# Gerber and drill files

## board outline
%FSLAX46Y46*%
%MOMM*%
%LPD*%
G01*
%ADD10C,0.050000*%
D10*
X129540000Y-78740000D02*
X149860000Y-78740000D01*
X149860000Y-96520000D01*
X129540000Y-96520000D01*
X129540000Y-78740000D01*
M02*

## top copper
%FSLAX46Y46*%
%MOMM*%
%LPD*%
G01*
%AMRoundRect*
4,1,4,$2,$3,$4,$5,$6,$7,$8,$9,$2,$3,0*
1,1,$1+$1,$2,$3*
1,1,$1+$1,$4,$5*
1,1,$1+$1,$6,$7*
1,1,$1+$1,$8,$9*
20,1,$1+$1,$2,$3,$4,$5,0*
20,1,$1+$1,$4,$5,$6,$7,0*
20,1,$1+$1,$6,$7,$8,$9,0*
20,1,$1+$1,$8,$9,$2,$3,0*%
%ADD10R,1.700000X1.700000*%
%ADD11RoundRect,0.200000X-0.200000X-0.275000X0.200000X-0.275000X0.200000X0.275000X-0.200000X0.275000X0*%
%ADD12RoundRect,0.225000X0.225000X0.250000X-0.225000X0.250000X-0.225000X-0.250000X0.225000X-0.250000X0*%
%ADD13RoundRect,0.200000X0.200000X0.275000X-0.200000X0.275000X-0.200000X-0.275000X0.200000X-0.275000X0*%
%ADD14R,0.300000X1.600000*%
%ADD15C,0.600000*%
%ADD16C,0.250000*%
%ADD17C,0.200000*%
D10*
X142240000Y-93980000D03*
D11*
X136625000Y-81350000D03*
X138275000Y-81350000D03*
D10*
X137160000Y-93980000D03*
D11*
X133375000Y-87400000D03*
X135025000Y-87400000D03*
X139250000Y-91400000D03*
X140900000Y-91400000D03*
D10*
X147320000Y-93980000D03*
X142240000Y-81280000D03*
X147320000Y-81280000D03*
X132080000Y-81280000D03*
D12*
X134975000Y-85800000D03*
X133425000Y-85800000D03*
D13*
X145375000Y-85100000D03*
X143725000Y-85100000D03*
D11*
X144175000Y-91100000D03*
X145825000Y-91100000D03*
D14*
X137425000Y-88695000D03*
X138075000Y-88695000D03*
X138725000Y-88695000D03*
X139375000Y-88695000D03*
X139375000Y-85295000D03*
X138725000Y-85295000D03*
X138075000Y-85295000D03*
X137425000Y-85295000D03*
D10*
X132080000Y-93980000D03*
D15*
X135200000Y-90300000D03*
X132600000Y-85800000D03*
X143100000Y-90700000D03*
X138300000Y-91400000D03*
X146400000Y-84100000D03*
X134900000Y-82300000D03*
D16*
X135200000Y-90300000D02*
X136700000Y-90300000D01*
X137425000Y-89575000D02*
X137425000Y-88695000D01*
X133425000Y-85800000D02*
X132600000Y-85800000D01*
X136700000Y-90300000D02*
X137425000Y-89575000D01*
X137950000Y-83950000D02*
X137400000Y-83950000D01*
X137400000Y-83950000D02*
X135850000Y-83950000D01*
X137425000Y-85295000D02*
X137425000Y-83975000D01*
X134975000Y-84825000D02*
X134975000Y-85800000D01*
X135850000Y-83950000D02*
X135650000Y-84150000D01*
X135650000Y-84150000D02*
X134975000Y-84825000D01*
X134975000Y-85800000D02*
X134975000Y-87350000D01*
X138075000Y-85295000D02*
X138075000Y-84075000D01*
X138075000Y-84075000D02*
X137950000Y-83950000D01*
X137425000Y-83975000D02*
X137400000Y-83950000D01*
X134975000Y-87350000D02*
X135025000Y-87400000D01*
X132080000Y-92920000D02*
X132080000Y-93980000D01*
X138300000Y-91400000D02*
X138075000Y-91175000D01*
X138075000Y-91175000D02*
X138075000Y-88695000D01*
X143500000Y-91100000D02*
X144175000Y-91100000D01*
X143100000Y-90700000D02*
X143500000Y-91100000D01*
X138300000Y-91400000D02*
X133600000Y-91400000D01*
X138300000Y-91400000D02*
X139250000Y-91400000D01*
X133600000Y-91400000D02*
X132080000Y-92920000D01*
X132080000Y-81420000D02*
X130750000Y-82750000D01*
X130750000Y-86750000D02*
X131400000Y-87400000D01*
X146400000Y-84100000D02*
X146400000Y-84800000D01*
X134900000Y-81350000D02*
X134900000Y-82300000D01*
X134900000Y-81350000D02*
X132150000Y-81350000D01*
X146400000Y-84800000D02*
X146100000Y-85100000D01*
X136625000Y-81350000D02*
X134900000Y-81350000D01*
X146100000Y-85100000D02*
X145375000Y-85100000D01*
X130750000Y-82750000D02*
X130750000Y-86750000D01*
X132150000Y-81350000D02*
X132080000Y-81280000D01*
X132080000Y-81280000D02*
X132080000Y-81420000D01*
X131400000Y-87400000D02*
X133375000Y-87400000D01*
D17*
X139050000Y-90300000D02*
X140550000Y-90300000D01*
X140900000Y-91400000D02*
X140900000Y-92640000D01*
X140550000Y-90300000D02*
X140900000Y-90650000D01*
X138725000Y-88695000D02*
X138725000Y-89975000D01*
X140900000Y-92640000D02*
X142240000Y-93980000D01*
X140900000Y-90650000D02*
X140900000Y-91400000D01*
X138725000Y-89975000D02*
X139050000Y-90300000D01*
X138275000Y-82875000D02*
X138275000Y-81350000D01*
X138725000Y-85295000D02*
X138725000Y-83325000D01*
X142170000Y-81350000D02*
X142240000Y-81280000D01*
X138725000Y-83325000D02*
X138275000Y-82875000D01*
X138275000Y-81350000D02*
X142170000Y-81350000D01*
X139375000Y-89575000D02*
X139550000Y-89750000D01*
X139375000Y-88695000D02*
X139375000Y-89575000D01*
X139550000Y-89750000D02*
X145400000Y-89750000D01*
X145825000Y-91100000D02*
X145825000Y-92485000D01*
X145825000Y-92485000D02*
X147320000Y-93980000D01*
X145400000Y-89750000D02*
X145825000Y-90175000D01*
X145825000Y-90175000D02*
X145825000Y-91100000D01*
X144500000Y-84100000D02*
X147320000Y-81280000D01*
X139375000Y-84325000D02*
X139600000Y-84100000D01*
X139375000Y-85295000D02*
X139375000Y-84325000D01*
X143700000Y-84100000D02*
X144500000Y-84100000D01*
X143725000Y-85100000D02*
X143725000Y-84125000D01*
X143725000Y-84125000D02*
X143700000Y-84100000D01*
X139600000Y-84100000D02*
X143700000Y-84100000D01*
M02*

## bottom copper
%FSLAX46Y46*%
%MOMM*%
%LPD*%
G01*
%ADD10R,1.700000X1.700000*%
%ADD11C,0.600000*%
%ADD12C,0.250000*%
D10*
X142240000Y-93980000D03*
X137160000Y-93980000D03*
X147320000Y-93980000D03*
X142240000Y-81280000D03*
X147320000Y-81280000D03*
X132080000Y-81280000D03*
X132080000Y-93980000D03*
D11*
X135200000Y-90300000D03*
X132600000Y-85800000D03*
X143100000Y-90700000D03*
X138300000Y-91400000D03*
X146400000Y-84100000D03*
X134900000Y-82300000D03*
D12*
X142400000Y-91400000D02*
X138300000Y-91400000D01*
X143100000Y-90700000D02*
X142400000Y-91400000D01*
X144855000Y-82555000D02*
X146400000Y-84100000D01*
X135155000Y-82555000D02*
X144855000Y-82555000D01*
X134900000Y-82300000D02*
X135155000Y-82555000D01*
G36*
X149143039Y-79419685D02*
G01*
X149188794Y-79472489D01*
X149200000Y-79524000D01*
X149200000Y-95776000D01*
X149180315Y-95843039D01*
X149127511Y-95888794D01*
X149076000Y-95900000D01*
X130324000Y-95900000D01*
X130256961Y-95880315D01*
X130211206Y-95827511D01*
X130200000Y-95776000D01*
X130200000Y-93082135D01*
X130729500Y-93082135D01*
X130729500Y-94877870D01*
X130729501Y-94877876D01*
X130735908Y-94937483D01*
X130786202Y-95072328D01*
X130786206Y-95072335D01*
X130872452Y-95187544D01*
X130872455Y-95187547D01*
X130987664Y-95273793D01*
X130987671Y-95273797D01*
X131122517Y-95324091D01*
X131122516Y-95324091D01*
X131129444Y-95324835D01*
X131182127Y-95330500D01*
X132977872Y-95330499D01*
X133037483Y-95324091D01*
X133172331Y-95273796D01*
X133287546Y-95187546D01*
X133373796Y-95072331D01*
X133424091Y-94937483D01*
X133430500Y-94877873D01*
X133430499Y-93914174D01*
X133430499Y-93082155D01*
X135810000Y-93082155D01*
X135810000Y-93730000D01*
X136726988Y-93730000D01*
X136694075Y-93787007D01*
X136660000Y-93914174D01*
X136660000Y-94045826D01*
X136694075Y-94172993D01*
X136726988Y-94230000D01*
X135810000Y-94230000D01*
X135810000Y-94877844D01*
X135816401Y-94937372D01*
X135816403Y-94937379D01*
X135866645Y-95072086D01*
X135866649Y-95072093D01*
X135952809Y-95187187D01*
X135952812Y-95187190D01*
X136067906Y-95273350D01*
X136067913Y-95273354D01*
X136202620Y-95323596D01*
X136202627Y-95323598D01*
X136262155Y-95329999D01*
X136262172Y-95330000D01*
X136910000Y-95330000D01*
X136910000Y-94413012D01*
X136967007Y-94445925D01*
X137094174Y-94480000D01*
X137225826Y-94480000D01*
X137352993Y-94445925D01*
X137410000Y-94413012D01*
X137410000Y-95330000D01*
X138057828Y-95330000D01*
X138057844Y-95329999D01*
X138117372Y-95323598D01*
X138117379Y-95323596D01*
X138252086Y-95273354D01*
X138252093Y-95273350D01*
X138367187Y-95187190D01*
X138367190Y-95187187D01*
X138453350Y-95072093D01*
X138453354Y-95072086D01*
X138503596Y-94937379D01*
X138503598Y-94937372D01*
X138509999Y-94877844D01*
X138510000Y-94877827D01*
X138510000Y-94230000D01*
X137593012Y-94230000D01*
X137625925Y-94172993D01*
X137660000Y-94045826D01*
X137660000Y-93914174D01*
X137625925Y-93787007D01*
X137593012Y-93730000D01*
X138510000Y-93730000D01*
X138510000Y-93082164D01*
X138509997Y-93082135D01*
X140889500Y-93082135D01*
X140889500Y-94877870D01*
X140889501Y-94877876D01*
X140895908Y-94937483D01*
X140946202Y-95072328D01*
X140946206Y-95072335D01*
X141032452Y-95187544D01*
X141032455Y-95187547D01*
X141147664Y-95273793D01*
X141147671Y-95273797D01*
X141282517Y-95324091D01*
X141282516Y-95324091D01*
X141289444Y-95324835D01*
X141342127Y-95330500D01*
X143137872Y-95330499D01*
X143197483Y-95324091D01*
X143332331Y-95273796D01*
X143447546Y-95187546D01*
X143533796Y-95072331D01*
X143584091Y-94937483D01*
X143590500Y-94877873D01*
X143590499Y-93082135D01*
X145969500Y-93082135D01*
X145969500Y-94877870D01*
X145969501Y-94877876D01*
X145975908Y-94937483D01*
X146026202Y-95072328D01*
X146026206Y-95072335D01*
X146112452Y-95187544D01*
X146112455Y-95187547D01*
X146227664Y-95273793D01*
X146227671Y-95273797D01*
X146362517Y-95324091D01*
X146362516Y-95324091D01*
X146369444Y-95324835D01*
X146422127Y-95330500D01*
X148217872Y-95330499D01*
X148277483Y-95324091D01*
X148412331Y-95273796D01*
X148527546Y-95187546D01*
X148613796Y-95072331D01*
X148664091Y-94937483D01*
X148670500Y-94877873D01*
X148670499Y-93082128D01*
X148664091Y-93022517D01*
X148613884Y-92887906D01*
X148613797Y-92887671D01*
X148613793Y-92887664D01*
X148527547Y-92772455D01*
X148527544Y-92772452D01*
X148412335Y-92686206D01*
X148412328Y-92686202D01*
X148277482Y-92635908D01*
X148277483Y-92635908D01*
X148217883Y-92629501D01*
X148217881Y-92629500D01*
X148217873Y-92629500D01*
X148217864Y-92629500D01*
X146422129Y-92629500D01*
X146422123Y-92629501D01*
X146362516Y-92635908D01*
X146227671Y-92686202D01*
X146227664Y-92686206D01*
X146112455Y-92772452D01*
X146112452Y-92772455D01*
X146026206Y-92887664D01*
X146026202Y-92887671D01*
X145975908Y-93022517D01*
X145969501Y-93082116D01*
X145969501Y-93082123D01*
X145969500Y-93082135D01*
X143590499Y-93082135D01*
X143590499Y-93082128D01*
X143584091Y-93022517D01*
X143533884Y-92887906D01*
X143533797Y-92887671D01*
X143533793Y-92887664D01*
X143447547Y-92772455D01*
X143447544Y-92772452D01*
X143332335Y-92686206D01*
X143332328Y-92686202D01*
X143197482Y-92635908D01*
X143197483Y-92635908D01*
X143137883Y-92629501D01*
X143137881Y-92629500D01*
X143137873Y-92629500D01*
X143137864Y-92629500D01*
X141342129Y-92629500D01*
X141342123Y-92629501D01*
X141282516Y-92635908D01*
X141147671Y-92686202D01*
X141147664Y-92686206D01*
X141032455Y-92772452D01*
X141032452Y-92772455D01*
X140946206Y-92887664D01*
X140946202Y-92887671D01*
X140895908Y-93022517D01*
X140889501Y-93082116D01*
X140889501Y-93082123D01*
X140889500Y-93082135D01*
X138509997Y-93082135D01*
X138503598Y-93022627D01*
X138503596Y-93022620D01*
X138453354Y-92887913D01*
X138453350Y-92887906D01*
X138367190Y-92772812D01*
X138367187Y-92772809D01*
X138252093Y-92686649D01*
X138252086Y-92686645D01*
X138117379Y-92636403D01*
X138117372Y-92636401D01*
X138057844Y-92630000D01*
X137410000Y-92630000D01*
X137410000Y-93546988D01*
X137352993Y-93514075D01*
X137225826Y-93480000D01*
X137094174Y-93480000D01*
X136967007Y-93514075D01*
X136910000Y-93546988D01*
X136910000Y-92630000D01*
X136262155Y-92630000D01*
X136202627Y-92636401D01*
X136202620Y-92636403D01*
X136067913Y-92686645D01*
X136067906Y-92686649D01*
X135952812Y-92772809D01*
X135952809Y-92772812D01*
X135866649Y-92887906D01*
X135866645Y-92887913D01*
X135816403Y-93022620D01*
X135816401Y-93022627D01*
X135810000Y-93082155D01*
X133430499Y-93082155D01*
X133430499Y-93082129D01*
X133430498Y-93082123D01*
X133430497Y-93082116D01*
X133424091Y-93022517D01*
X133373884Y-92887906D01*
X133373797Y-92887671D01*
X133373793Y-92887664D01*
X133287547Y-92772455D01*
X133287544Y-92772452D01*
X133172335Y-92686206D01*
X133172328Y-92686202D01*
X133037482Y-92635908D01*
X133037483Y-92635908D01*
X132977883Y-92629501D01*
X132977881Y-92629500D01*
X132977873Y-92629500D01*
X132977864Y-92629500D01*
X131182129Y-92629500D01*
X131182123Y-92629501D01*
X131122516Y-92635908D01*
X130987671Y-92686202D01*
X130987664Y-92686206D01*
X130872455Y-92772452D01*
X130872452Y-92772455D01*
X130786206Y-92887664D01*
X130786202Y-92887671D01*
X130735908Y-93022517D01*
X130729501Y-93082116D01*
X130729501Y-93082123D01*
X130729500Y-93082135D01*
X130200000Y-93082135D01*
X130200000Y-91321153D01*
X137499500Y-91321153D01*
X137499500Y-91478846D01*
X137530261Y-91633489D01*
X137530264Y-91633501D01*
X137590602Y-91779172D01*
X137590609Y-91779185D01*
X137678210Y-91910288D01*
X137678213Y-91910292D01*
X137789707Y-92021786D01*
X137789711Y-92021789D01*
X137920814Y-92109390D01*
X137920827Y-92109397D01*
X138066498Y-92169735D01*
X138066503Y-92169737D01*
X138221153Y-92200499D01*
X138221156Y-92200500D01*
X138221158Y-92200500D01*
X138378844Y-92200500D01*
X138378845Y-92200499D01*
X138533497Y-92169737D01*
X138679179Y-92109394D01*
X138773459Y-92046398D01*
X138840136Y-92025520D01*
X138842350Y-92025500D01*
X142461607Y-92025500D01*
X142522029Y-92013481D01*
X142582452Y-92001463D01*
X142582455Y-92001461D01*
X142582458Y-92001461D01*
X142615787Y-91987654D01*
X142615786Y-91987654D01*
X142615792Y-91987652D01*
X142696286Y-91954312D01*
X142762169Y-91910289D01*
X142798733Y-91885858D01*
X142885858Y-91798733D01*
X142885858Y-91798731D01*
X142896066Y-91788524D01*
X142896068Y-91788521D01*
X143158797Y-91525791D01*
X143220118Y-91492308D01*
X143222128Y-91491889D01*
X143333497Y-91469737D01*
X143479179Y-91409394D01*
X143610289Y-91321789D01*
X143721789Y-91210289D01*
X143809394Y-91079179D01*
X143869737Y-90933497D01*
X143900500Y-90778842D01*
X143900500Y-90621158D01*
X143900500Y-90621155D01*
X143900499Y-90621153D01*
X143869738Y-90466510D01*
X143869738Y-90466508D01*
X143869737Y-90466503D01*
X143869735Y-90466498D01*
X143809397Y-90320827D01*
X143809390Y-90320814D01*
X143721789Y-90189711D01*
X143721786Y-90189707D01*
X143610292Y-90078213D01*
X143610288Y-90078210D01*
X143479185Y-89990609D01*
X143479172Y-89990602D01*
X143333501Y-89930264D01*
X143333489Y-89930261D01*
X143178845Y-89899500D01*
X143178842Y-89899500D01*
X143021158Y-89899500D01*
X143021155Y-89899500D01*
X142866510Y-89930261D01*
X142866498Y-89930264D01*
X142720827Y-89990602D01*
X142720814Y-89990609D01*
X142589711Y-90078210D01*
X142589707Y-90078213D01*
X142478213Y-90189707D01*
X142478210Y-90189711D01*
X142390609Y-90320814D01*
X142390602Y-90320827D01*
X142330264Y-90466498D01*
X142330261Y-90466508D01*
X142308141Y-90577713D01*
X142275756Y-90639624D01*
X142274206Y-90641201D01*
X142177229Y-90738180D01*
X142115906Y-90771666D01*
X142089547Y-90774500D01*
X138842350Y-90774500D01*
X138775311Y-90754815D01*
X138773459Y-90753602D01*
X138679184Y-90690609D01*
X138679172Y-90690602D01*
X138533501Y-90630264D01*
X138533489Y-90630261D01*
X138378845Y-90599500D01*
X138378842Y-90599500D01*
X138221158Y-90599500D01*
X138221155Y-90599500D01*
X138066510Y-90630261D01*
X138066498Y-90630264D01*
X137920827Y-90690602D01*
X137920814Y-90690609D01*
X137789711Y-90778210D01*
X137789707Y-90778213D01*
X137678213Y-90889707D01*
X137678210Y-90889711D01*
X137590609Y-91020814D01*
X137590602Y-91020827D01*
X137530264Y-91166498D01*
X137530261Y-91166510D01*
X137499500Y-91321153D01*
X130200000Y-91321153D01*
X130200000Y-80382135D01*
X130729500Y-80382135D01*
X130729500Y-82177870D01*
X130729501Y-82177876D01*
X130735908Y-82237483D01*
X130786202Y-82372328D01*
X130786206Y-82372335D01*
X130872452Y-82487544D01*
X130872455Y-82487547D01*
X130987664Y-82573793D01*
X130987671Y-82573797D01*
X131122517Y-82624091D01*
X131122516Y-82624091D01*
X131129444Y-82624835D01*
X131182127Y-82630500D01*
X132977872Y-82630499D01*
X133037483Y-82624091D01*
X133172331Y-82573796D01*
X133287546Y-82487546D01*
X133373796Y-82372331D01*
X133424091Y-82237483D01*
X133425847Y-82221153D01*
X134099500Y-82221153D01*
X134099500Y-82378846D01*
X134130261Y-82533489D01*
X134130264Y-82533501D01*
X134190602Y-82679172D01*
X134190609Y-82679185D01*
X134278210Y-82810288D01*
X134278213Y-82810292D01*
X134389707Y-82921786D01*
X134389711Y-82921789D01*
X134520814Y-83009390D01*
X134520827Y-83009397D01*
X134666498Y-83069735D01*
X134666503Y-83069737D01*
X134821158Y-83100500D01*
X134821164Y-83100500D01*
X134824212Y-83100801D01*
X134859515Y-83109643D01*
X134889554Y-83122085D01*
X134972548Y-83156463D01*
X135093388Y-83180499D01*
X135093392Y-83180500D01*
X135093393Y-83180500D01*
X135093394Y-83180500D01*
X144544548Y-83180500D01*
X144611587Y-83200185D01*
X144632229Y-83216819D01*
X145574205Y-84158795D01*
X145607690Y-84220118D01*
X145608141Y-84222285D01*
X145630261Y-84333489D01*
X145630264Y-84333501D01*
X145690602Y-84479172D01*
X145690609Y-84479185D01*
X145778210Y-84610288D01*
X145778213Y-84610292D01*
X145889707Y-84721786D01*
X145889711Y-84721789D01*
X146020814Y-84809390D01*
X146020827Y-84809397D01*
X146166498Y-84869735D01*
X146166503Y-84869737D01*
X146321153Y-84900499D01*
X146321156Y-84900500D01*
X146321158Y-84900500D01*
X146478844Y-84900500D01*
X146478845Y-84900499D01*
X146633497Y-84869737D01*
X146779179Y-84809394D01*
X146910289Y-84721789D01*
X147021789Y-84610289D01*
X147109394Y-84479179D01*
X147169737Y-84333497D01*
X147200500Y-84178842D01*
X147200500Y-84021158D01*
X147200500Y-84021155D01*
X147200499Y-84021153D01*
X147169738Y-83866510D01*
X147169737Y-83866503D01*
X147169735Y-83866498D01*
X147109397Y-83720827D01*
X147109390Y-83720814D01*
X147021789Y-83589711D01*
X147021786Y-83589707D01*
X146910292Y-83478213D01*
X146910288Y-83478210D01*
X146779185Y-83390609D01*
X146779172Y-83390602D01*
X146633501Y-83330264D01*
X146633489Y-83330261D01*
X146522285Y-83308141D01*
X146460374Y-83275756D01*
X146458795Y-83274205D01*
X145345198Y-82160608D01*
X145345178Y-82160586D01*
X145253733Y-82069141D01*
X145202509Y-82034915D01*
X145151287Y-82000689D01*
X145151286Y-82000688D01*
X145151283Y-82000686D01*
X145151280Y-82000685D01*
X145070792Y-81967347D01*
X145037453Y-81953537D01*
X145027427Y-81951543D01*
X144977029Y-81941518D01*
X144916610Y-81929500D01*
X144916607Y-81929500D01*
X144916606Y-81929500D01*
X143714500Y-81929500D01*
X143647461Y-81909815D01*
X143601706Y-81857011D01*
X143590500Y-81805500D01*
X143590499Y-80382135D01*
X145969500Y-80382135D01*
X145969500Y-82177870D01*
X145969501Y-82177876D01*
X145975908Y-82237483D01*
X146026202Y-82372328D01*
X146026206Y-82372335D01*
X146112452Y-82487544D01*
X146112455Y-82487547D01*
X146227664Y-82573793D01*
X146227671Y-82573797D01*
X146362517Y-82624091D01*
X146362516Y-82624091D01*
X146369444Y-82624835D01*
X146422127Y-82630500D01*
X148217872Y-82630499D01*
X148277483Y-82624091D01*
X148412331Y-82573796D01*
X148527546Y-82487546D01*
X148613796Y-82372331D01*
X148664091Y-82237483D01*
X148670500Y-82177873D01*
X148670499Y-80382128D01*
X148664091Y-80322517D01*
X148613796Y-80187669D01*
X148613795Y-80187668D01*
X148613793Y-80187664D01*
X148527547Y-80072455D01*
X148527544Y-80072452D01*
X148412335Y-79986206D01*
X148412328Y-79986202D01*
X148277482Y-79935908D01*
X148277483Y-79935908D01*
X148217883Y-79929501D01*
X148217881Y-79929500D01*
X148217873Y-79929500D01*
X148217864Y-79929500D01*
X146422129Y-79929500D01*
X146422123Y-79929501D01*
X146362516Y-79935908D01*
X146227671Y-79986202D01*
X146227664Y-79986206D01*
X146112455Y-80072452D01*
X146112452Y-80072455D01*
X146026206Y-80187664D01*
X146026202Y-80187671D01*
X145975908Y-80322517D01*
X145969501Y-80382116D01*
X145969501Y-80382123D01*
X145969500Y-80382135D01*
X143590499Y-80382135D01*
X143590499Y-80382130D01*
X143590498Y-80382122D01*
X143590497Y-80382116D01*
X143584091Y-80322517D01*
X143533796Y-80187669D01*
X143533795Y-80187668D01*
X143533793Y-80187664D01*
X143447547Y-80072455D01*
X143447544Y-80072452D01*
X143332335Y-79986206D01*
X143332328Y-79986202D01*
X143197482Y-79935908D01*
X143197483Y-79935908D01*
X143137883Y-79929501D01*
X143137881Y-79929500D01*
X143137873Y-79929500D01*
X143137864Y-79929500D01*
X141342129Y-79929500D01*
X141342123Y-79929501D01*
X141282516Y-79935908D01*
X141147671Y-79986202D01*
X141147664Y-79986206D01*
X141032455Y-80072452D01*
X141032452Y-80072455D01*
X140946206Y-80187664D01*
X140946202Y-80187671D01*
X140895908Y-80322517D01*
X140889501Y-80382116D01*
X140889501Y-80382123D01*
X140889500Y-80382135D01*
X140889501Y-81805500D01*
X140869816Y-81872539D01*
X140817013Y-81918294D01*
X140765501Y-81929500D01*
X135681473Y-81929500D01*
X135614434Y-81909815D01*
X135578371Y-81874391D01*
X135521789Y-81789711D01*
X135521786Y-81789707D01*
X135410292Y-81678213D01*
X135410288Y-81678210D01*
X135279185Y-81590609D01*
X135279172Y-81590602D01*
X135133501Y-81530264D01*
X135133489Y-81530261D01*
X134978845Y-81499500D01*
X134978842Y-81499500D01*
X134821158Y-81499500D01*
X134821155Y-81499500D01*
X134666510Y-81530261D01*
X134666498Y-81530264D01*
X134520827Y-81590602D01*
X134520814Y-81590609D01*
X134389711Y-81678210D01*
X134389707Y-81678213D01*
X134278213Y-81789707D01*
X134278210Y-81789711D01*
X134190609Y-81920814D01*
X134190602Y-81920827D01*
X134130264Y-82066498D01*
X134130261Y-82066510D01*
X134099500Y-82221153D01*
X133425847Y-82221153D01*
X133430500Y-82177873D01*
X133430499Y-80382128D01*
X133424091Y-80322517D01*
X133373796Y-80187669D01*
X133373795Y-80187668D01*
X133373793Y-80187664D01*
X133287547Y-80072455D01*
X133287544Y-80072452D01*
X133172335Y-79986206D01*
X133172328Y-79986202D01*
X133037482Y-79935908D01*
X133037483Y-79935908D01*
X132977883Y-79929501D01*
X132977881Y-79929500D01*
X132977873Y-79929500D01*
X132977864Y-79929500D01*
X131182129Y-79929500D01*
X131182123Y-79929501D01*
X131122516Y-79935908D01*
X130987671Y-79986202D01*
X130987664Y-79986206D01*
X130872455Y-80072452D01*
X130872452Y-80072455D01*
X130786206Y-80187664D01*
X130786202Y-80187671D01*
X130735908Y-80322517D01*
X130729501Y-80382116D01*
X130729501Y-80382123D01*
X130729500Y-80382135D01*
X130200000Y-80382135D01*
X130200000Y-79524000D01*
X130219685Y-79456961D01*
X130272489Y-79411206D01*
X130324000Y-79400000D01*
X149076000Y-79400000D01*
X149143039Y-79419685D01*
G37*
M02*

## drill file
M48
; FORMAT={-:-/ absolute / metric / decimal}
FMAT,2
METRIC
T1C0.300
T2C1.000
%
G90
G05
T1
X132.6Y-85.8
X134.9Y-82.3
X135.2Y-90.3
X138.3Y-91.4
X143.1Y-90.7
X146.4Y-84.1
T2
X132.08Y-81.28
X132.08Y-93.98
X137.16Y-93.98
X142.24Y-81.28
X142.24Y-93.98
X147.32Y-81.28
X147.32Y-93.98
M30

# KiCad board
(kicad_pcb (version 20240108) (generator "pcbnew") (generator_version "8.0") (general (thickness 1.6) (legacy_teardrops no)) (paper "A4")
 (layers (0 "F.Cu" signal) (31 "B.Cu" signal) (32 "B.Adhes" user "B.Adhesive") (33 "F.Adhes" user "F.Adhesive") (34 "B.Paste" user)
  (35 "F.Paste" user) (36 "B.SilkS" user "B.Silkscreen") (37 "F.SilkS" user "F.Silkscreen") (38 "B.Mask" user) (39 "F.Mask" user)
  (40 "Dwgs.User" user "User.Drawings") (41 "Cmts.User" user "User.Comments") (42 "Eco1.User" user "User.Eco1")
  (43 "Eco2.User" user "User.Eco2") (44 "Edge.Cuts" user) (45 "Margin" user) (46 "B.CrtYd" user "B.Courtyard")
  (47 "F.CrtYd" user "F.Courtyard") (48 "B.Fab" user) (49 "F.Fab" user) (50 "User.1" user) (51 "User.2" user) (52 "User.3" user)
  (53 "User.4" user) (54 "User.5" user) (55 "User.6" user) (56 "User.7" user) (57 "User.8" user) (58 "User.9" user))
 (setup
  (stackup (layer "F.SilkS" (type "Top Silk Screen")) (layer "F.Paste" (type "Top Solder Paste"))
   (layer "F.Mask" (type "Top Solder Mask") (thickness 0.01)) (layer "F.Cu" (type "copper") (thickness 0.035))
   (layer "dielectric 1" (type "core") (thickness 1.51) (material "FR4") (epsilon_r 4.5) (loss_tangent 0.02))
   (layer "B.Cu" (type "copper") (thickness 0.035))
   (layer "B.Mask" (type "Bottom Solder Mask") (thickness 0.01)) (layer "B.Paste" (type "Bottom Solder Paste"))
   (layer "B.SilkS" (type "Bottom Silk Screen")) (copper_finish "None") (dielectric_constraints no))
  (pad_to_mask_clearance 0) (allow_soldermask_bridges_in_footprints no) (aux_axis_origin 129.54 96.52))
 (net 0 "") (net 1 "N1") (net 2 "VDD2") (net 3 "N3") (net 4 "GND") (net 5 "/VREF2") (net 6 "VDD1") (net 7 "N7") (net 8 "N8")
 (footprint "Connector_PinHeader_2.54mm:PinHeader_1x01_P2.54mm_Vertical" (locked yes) (layer "F.Cu") (at 142.24 93.98)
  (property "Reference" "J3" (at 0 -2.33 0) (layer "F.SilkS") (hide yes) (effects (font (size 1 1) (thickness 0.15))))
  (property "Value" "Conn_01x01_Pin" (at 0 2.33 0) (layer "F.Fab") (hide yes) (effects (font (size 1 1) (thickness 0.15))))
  (pad "1" thru_hole rect (at 0 0) (size 1.7 1.7) (drill 1) (layers "*.Cu" "*.Mask") (remove_unused_layers no) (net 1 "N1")))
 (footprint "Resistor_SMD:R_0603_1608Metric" (layer "F.Cu") (at 137.45 81.35)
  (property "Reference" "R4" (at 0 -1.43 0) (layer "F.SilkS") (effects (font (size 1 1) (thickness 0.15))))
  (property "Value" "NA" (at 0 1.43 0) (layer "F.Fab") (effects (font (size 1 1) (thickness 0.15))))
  (pad "1" smd roundrect (at -0.825 0) (size 0.8 0.95) (layers "F.Cu" "F.Paste" "F.Mask") (roundrect_rratio 0.25) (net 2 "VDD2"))
  (pad "2" smd roundrect (at 0.825 0) (size 0.8 0.95) (layers "F.Cu" "F.Paste" "F.Mask") (roundrect_rratio 0.25) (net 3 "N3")))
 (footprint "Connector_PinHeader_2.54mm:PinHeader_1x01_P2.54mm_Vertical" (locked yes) (layer "F.Cu") (at 137.16 93.98)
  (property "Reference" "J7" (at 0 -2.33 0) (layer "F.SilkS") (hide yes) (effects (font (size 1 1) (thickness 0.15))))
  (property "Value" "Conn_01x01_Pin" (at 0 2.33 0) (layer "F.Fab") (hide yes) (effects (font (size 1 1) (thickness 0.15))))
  (pad "1" thru_hole rect (at 0 0) (size 1.7 1.7) (drill 1) (layers "*.Cu" "*.Mask") (remove_unused_layers no) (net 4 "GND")))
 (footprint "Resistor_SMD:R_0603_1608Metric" (layer "F.Cu") (at 134.2 87.4)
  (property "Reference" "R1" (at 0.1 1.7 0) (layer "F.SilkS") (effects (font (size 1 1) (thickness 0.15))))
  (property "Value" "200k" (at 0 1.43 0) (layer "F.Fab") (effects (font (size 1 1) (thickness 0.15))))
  (pad "1" smd roundrect (at -0.825 0) (size 0.8 0.95) (layers "F.Cu" "F.Paste" "F.Mask") (roundrect_rratio 0.25) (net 2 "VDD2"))
  (pad "2" smd roundrect (at 0.825 0) (size 0.8 0.95) (layers "F.Cu" "F.Paste" "F.Mask") (roundrect_rratio 0.25) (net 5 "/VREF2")))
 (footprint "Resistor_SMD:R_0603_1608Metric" (layer "F.Cu") (at 140.075 91.4)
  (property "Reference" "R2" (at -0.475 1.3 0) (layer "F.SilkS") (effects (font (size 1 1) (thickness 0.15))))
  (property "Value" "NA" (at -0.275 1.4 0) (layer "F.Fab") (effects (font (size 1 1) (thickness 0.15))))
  (pad "1" smd roundrect (at -0.825 0) (size 0.8 0.95) (layers "F.Cu" "F.Paste" "F.Mask") (roundrect_rratio 0.25) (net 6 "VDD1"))
  (pad "2" smd roundrect (at 0.825 0) (size 0.8 0.95) (layers "F.Cu" "F.Paste" "F.Mask") (roundrect_rratio 0.25) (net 1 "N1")))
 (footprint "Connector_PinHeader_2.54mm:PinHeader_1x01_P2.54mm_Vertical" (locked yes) (layer "F.Cu") (at 147.32 93.98)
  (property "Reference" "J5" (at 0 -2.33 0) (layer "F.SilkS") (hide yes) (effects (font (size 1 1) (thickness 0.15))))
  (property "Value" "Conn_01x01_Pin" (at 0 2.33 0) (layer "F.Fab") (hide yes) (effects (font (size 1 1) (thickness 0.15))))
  (pad "1" thru_hole rect (at 0 0) (size 1.7 1.7) (drill 1) (layers "*.Cu" "*.Mask") (remove_unused_layers no) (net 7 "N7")))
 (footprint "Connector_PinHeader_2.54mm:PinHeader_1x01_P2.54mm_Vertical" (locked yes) (layer "F.Cu") (at 142.24 81.28)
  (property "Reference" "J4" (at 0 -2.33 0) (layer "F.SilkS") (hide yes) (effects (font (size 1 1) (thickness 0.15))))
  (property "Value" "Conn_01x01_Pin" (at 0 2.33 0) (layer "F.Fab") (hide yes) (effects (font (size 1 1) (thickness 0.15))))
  (pad "1" thru_hole rect (at 0 0) (size 1.7 1.7) (drill 1) (layers "*.Cu" "*.Mask") (remove_unused_layers no) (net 3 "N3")))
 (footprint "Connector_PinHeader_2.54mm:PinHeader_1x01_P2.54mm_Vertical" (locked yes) (layer "F.Cu") (at 147.32 81.28)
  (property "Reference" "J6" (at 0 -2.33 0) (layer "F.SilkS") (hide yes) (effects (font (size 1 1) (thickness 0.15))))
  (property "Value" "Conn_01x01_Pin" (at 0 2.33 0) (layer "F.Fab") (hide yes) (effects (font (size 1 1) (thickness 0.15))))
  (pad "1" thru_hole rect (at 0 0) (size 1.7 1.7) (drill 1) (layers "*.Cu" "*.Mask") (remove_unused_layers no) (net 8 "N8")))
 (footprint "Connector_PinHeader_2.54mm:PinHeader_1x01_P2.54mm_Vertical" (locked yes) (layer "F.Cu") (at 132.08 81.28)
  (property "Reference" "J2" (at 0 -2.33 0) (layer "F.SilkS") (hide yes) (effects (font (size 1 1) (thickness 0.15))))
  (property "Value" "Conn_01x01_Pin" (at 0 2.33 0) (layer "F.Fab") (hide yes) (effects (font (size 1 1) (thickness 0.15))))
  (pad "1" thru_hole rect (at 0 0) (size 1.7 1.7) (drill 1) (layers "*.Cu" "*.Mask") (remove_unused_layers no) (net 2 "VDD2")))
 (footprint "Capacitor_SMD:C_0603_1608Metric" (layer "F.Cu") (at 134.2 85.8 180)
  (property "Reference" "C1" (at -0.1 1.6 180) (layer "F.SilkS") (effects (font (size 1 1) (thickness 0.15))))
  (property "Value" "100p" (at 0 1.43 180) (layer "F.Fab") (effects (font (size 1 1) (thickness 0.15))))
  (pad "1" smd roundrect (at -0.775 0 180) (size 0.9 0.95) (layers "F.Cu" "F.Paste" "F.Mask") (roundrect_rratio 0.25) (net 5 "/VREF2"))
  (pad "2" smd roundrect (at 0.775 0 180) (size 0.9 0.95) (layers "F.Cu" "F.Paste" "F.Mask") (roundrect_rratio 0.25) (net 4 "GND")))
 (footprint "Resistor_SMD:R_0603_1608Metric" (layer "F.Cu") (at 144.55 85.1 180)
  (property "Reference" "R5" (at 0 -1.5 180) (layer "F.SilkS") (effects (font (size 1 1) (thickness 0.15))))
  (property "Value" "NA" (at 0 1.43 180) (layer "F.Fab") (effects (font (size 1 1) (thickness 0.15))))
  (pad "1" smd roundrect (at -0.825 0 180) (size 0.8 0.95) (layers "F.Cu" "F.Paste" "F.Mask") (roundrect_rratio 0.25) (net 2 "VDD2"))
  (pad "2" smd roundrect (at 0.825 0 180) (size 0.8 0.95) (layers "F.Cu" "F.Paste" "F.Mask") (roundrect_rratio 0.25) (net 8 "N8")))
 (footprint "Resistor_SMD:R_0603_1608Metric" (layer "F.Cu") (at 145 91.1)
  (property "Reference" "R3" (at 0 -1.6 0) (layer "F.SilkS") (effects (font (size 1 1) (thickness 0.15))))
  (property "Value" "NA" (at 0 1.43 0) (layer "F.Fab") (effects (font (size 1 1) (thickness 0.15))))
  (pad "1" smd roundrect (at -0.825 0) (size 0.8 0.95) (layers "F.Cu" "F.Paste" "F.Mask") (roundrect_rratio 0.25) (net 6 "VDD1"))
  (pad "2" smd roundrect (at 0.825 0) (size 0.8 0.95) (layers "F.Cu" "F.Paste" "F.Mask") (roundrect_rratio 0.25) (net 7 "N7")))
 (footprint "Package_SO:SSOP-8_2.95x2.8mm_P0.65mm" (layer "F.Cu") (at 138.4 86.995 90)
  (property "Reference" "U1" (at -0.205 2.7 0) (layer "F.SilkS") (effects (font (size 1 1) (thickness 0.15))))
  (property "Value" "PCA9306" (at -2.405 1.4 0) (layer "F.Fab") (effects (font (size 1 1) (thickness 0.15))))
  (pad "1" smd rect (at -1.7 -0.975) (size 0.3 1.6) (layers "F.Cu" "F.Paste" "F.Mask") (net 4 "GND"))
  (pad "2" smd rect (at -1.7 -0.325) (size 0.3 1.6) (layers "F.Cu" "F.Paste" "F.Mask") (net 6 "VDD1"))
  (pad "3" smd rect (at -1.7 0.325) (size 0.3 1.6) (layers "F.Cu" "F.Paste" "F.Mask") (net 1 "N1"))
  (pad "4" smd rect (at -1.7 0.975) (size 0.3 1.6) (layers "F.Cu" "F.Paste" "F.Mask") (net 7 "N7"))
  (pad "5" smd rect (at 1.7 0.975) (size 0.3 1.6) (layers "F.Cu" "F.Paste" "F.Mask") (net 8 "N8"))
  (pad "6" smd rect (at 1.7 0.325) (size 0.3 1.6) (layers "F.Cu" "F.Paste" "F.Mask") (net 3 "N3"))
  (pad "7" smd rect (at 1.7 -0.325) (size 0.3 1.6) (layers "F.Cu" "F.Paste" "F.Mask") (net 5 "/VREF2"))
  (pad "8" smd rect (at 1.7 -0.975) (size 0.3 1.6) (layers "F.Cu" "F.Paste" "F.Mask") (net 5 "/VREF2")))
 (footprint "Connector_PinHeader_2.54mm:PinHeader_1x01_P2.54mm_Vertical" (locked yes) (layer "F.Cu") (at 132.08 93.98)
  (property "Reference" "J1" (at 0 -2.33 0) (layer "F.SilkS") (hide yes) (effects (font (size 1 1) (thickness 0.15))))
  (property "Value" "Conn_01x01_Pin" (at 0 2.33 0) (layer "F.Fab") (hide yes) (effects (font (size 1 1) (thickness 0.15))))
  (pad "1" thru_hole rect (at 0 0) (size 1.7 1.7) (drill 1) (layers "*.Cu" "*.Mask") (remove_unused_layers no) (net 6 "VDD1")))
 (gr_rect (start 129.54 78.74) (end 149.86 96.52) (stroke (width 0.05) (type default)) (fill none) (layer "Edge.Cuts"))
 (segment (start 135.2 90.3) (end 136.7 90.3) (width 0.25) (layer "F.Cu") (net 4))
 (segment (start 137.425 89.575) (end 137.425 88.695) (width 0.25) (layer "F.Cu") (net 4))
 (segment (start 133.425 85.8) (end 132.6 85.8) (width 0.25) (layer "F.Cu") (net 4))
 (segment (start 136.7 90.3) (end 137.425 89.575) (width 0.25) (layer "F.Cu") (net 4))
 (via (at 135.2 90.3) (size 0.6) (drill 0.3) (layers "F.Cu" "B.Cu") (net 4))
 (via (at 132.6 85.8) (size 0.6) (drill 0.3) (layers "F.Cu" "B.Cu") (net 4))
 (segment (start 137.95 83.95) (end 137.4 83.95) (width 0.25) (layer "F.Cu") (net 5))
 (segment (start 137.4 83.95) (end 135.85 83.95) (width 0.25) (layer "F.Cu") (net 5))
 (segment (start 137.425 85.295) (end 137.425 83.975) (width 0.25) (layer "F.Cu") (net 5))
 (segment (start 134.975 84.825) (end 134.975 85.8) (width 0.25) (layer "F.Cu") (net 5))
 (segment (start 135.85 83.95) (end 135.65 84.15) (width 0.25) (layer "F.Cu") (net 5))
 (segment (start 135.65 84.15) (end 134.975 84.825) (width 0.25) (layer "F.Cu") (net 5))
 (segment (start 134.975 85.8) (end 134.975 87.35) (width 0.25) (layer "F.Cu") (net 5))
 (segment (start 138.075 85.295) (end 138.075 84.075) (width 0.25) (layer "F.Cu") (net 5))
 (segment (start 138.075 84.075) (end 137.95 83.95) (width 0.25) (layer "F.Cu") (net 5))
 (segment (start 137.425 83.975) (end 137.4 83.95) (width 0.25) (layer "F.Cu") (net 5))
 (segment (start 134.975 87.35) (end 135.025 87.4) (width 0.25) (layer "F.Cu") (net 5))
 (segment (start 132.08 92.92) (end 132.08 93.98) (width 0.25) (layer "F.Cu") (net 6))
 (segment (start 138.3 91.4) (end 138.075 91.175) (width 0.25) (layer "F.Cu") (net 6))
 (segment (start 138.075 91.175) (end 138.075 88.695) (width 0.25) (layer "F.Cu") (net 6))
 (segment (start 143.5 91.1) (end 144.175 91.1) (width 0.25) (layer "F.Cu") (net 6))
 (segment (start 143.1 90.7) (end 143.5 91.1) (width 0.25) (layer "F.Cu") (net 6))
 (segment (start 138.3 91.4) (end 133.6 91.4) (width 0.25) (layer "F.Cu") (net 6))
 (segment (start 138.3 91.4) (end 139.25 91.4) (width 0.25) (layer "F.Cu") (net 6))
 (segment (start 133.6 91.4) (end 132.08 92.92) (width 0.25) (layer "F.Cu") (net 6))
 (via (at 143.1 90.7) (size 0.6) (drill 0.3) (layers "F.Cu" "B.Cu") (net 6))
 (via (at 138.3 91.4) (size 0.6) (drill 0.3) (layers "F.Cu" "B.Cu") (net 6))
 (segment (start 142.4 91.4) (end 138.3 91.4) (width 0.25) (layer "B.Cu") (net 6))
 (segment (start 143.1 90.7) (end 142.4 91.4) (width 0.25) (layer "B.Cu") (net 6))
 (segment (start 132.08 81.42) (end 130.75 82.75) (width 0.25) (layer "F.Cu") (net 2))
 (segment (start 130.75 86.75) (end 131.4 87.4) (width 0.25) (layer "F.Cu") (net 2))
 (segment (start 146.4 84.1) (end 146.4 84.8) (width 0.25) (layer "F.Cu") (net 2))
 (segment (start 134.9 81.35) (end 134.9 82.3) (width 0.25) (layer "F.Cu") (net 2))
 (segment (start 134.9 81.35) (end 132.15 81.35) (width 0.25) (layer "F.Cu") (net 2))
 (segment (start 146.4 84.8) (end 146.1 85.1) (width 0.25) (layer "F.Cu") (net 2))
 (segment (start 136.625 81.35) (end 134.9 81.35) (width 0.25) (layer "F.Cu") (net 2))
 (segment (start 146.1 85.1) (end 145.375 85.1) (width 0.25) (layer "F.Cu") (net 2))
 (segment (start 130.75 82.75) (end 130.75 86.75) (width 0.25) (layer "F.Cu") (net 2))
 (segment (start 132.15 81.35) (end 132.08 81.28) (width 0.25) (layer "F.Cu") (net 2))
 (segment (start 132.08 81.28) (end 132.08 81.42) (width 0.25) (layer "F.Cu") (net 2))
 (segment (start 131.4 87.4) (end 133.375 87.4) (width 0.25) (layer "F.Cu") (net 2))
 (via (at 146.4 84.1) (size 0.6) (drill 0.3) (layers "F.Cu" "B.Cu") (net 2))
 (via (at 134.9 82.3) (size 0.6) (drill 0.3) (layers "F.Cu" "B.Cu") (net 2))
 (segment (start 144.855 82.555) (end 146.4 84.1) (width 0.25) (layer "B.Cu") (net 2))
 (segment (start 135.155 82.555) (end 144.855 82.555) (width 0.25) (layer "B.Cu") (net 2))
 (segment (start 134.9 82.3) (end 135.155 82.555) (width 0.25) (layer "B.Cu") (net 2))
 (segment (start 139.05 90.3) (end 140.55 90.3) (width 0.2) (layer "F.Cu") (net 1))
 (segment (start 140.9 91.4) (end 140.9 92.64) (width 0.2) (layer "F.Cu") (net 1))
 (segment (start 140.55 90.3) (end 140.9 90.65) (width 0.2) (layer "F.Cu") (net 1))
 (segment (start 138.725 88.695) (end 138.725 89.975) (width 0.2) (layer "F.Cu") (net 1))
 (segment (start 140.9 92.64) (end 142.24 93.98) (width 0.2) (layer "F.Cu") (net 1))
 (segment (start 140.9 90.65) (end 140.9 91.4) (width 0.2) (layer "F.Cu") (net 1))
 (segment (start 138.725 89.975) (end 139.05 90.3) (width 0.2) (layer "F.Cu") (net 1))
 (segment (start 138.275 82.875) (end 138.275 81.35) (width 0.2) (layer "F.Cu") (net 3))
 (segment (start 138.725 85.295) (end 138.725 83.325) (width 0.2) (layer "F.Cu") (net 3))
 (segment (start 142.17 81.35) (end 142.24 81.28) (width 0.2) (layer "F.Cu") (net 3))
 (segment (start 138.725 83.325) (end 138.275 82.875) (width 0.2) (layer "F.Cu") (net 3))
 (segment (start 138.275 81.35) (end 142.17 81.35) (width 0.2) (layer "F.Cu") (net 3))
 (segment (start 139.375 89.575) (end 139.55 89.75) (width 0.2) (layer "F.Cu") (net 7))
 (segment (start 139.375 88.695) (end 139.375 89.575) (width 0.2) (layer "F.Cu") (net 7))
 (segment (start 139.55 89.75) (end 145.4 89.75) (width 0.2) (layer "F.Cu") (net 7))
 (segment (start 145.825 91.1) (end 145.825 92.485) (width 0.2) (layer "F.Cu") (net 7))
 (segment (start 145.825 92.485) (end 147.32 93.98) (width 0.2) (layer "F.Cu") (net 7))
 (segment (start 145.4 89.75) (end 145.825 90.175) (width 0.2) (layer "F.Cu") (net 7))
 (segment (start 145.825 90.175) (end 145.825 91.1) (width 0.2) (layer "F.Cu") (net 7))
 (segment (start 144.5 84.1) (end 147.32 81.28) (width 0.2) (layer "F.Cu") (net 8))
 (segment (start 139.375 84.325) (end 139.6 84.1) (width 0.2) (layer "F.Cu") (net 8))
 (segment (start 139.375 85.295) (end 139.375 84.325) (width 0.2) (layer "F.Cu") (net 8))
 (segment (start 143.7 84.1) (end 144.5 84.1) (width 0.2) (layer "F.Cu") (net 8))
 (segment (start 143.725 85.1) (end 143.725 84.125) (width 0.2) (layer "F.Cu") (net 8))
 (segment (start 143.725 84.125) (end 143.7 84.1) (width 0.2) (layer "F.Cu") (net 8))
 (segment (start 139.6 84.1) (end 143.7 84.1) (width 0.2) (layer "F.Cu") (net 8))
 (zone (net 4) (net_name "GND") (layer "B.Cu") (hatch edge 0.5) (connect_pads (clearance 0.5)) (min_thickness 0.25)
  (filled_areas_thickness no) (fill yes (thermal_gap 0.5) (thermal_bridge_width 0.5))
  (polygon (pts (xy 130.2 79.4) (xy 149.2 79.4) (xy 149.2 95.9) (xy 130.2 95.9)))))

